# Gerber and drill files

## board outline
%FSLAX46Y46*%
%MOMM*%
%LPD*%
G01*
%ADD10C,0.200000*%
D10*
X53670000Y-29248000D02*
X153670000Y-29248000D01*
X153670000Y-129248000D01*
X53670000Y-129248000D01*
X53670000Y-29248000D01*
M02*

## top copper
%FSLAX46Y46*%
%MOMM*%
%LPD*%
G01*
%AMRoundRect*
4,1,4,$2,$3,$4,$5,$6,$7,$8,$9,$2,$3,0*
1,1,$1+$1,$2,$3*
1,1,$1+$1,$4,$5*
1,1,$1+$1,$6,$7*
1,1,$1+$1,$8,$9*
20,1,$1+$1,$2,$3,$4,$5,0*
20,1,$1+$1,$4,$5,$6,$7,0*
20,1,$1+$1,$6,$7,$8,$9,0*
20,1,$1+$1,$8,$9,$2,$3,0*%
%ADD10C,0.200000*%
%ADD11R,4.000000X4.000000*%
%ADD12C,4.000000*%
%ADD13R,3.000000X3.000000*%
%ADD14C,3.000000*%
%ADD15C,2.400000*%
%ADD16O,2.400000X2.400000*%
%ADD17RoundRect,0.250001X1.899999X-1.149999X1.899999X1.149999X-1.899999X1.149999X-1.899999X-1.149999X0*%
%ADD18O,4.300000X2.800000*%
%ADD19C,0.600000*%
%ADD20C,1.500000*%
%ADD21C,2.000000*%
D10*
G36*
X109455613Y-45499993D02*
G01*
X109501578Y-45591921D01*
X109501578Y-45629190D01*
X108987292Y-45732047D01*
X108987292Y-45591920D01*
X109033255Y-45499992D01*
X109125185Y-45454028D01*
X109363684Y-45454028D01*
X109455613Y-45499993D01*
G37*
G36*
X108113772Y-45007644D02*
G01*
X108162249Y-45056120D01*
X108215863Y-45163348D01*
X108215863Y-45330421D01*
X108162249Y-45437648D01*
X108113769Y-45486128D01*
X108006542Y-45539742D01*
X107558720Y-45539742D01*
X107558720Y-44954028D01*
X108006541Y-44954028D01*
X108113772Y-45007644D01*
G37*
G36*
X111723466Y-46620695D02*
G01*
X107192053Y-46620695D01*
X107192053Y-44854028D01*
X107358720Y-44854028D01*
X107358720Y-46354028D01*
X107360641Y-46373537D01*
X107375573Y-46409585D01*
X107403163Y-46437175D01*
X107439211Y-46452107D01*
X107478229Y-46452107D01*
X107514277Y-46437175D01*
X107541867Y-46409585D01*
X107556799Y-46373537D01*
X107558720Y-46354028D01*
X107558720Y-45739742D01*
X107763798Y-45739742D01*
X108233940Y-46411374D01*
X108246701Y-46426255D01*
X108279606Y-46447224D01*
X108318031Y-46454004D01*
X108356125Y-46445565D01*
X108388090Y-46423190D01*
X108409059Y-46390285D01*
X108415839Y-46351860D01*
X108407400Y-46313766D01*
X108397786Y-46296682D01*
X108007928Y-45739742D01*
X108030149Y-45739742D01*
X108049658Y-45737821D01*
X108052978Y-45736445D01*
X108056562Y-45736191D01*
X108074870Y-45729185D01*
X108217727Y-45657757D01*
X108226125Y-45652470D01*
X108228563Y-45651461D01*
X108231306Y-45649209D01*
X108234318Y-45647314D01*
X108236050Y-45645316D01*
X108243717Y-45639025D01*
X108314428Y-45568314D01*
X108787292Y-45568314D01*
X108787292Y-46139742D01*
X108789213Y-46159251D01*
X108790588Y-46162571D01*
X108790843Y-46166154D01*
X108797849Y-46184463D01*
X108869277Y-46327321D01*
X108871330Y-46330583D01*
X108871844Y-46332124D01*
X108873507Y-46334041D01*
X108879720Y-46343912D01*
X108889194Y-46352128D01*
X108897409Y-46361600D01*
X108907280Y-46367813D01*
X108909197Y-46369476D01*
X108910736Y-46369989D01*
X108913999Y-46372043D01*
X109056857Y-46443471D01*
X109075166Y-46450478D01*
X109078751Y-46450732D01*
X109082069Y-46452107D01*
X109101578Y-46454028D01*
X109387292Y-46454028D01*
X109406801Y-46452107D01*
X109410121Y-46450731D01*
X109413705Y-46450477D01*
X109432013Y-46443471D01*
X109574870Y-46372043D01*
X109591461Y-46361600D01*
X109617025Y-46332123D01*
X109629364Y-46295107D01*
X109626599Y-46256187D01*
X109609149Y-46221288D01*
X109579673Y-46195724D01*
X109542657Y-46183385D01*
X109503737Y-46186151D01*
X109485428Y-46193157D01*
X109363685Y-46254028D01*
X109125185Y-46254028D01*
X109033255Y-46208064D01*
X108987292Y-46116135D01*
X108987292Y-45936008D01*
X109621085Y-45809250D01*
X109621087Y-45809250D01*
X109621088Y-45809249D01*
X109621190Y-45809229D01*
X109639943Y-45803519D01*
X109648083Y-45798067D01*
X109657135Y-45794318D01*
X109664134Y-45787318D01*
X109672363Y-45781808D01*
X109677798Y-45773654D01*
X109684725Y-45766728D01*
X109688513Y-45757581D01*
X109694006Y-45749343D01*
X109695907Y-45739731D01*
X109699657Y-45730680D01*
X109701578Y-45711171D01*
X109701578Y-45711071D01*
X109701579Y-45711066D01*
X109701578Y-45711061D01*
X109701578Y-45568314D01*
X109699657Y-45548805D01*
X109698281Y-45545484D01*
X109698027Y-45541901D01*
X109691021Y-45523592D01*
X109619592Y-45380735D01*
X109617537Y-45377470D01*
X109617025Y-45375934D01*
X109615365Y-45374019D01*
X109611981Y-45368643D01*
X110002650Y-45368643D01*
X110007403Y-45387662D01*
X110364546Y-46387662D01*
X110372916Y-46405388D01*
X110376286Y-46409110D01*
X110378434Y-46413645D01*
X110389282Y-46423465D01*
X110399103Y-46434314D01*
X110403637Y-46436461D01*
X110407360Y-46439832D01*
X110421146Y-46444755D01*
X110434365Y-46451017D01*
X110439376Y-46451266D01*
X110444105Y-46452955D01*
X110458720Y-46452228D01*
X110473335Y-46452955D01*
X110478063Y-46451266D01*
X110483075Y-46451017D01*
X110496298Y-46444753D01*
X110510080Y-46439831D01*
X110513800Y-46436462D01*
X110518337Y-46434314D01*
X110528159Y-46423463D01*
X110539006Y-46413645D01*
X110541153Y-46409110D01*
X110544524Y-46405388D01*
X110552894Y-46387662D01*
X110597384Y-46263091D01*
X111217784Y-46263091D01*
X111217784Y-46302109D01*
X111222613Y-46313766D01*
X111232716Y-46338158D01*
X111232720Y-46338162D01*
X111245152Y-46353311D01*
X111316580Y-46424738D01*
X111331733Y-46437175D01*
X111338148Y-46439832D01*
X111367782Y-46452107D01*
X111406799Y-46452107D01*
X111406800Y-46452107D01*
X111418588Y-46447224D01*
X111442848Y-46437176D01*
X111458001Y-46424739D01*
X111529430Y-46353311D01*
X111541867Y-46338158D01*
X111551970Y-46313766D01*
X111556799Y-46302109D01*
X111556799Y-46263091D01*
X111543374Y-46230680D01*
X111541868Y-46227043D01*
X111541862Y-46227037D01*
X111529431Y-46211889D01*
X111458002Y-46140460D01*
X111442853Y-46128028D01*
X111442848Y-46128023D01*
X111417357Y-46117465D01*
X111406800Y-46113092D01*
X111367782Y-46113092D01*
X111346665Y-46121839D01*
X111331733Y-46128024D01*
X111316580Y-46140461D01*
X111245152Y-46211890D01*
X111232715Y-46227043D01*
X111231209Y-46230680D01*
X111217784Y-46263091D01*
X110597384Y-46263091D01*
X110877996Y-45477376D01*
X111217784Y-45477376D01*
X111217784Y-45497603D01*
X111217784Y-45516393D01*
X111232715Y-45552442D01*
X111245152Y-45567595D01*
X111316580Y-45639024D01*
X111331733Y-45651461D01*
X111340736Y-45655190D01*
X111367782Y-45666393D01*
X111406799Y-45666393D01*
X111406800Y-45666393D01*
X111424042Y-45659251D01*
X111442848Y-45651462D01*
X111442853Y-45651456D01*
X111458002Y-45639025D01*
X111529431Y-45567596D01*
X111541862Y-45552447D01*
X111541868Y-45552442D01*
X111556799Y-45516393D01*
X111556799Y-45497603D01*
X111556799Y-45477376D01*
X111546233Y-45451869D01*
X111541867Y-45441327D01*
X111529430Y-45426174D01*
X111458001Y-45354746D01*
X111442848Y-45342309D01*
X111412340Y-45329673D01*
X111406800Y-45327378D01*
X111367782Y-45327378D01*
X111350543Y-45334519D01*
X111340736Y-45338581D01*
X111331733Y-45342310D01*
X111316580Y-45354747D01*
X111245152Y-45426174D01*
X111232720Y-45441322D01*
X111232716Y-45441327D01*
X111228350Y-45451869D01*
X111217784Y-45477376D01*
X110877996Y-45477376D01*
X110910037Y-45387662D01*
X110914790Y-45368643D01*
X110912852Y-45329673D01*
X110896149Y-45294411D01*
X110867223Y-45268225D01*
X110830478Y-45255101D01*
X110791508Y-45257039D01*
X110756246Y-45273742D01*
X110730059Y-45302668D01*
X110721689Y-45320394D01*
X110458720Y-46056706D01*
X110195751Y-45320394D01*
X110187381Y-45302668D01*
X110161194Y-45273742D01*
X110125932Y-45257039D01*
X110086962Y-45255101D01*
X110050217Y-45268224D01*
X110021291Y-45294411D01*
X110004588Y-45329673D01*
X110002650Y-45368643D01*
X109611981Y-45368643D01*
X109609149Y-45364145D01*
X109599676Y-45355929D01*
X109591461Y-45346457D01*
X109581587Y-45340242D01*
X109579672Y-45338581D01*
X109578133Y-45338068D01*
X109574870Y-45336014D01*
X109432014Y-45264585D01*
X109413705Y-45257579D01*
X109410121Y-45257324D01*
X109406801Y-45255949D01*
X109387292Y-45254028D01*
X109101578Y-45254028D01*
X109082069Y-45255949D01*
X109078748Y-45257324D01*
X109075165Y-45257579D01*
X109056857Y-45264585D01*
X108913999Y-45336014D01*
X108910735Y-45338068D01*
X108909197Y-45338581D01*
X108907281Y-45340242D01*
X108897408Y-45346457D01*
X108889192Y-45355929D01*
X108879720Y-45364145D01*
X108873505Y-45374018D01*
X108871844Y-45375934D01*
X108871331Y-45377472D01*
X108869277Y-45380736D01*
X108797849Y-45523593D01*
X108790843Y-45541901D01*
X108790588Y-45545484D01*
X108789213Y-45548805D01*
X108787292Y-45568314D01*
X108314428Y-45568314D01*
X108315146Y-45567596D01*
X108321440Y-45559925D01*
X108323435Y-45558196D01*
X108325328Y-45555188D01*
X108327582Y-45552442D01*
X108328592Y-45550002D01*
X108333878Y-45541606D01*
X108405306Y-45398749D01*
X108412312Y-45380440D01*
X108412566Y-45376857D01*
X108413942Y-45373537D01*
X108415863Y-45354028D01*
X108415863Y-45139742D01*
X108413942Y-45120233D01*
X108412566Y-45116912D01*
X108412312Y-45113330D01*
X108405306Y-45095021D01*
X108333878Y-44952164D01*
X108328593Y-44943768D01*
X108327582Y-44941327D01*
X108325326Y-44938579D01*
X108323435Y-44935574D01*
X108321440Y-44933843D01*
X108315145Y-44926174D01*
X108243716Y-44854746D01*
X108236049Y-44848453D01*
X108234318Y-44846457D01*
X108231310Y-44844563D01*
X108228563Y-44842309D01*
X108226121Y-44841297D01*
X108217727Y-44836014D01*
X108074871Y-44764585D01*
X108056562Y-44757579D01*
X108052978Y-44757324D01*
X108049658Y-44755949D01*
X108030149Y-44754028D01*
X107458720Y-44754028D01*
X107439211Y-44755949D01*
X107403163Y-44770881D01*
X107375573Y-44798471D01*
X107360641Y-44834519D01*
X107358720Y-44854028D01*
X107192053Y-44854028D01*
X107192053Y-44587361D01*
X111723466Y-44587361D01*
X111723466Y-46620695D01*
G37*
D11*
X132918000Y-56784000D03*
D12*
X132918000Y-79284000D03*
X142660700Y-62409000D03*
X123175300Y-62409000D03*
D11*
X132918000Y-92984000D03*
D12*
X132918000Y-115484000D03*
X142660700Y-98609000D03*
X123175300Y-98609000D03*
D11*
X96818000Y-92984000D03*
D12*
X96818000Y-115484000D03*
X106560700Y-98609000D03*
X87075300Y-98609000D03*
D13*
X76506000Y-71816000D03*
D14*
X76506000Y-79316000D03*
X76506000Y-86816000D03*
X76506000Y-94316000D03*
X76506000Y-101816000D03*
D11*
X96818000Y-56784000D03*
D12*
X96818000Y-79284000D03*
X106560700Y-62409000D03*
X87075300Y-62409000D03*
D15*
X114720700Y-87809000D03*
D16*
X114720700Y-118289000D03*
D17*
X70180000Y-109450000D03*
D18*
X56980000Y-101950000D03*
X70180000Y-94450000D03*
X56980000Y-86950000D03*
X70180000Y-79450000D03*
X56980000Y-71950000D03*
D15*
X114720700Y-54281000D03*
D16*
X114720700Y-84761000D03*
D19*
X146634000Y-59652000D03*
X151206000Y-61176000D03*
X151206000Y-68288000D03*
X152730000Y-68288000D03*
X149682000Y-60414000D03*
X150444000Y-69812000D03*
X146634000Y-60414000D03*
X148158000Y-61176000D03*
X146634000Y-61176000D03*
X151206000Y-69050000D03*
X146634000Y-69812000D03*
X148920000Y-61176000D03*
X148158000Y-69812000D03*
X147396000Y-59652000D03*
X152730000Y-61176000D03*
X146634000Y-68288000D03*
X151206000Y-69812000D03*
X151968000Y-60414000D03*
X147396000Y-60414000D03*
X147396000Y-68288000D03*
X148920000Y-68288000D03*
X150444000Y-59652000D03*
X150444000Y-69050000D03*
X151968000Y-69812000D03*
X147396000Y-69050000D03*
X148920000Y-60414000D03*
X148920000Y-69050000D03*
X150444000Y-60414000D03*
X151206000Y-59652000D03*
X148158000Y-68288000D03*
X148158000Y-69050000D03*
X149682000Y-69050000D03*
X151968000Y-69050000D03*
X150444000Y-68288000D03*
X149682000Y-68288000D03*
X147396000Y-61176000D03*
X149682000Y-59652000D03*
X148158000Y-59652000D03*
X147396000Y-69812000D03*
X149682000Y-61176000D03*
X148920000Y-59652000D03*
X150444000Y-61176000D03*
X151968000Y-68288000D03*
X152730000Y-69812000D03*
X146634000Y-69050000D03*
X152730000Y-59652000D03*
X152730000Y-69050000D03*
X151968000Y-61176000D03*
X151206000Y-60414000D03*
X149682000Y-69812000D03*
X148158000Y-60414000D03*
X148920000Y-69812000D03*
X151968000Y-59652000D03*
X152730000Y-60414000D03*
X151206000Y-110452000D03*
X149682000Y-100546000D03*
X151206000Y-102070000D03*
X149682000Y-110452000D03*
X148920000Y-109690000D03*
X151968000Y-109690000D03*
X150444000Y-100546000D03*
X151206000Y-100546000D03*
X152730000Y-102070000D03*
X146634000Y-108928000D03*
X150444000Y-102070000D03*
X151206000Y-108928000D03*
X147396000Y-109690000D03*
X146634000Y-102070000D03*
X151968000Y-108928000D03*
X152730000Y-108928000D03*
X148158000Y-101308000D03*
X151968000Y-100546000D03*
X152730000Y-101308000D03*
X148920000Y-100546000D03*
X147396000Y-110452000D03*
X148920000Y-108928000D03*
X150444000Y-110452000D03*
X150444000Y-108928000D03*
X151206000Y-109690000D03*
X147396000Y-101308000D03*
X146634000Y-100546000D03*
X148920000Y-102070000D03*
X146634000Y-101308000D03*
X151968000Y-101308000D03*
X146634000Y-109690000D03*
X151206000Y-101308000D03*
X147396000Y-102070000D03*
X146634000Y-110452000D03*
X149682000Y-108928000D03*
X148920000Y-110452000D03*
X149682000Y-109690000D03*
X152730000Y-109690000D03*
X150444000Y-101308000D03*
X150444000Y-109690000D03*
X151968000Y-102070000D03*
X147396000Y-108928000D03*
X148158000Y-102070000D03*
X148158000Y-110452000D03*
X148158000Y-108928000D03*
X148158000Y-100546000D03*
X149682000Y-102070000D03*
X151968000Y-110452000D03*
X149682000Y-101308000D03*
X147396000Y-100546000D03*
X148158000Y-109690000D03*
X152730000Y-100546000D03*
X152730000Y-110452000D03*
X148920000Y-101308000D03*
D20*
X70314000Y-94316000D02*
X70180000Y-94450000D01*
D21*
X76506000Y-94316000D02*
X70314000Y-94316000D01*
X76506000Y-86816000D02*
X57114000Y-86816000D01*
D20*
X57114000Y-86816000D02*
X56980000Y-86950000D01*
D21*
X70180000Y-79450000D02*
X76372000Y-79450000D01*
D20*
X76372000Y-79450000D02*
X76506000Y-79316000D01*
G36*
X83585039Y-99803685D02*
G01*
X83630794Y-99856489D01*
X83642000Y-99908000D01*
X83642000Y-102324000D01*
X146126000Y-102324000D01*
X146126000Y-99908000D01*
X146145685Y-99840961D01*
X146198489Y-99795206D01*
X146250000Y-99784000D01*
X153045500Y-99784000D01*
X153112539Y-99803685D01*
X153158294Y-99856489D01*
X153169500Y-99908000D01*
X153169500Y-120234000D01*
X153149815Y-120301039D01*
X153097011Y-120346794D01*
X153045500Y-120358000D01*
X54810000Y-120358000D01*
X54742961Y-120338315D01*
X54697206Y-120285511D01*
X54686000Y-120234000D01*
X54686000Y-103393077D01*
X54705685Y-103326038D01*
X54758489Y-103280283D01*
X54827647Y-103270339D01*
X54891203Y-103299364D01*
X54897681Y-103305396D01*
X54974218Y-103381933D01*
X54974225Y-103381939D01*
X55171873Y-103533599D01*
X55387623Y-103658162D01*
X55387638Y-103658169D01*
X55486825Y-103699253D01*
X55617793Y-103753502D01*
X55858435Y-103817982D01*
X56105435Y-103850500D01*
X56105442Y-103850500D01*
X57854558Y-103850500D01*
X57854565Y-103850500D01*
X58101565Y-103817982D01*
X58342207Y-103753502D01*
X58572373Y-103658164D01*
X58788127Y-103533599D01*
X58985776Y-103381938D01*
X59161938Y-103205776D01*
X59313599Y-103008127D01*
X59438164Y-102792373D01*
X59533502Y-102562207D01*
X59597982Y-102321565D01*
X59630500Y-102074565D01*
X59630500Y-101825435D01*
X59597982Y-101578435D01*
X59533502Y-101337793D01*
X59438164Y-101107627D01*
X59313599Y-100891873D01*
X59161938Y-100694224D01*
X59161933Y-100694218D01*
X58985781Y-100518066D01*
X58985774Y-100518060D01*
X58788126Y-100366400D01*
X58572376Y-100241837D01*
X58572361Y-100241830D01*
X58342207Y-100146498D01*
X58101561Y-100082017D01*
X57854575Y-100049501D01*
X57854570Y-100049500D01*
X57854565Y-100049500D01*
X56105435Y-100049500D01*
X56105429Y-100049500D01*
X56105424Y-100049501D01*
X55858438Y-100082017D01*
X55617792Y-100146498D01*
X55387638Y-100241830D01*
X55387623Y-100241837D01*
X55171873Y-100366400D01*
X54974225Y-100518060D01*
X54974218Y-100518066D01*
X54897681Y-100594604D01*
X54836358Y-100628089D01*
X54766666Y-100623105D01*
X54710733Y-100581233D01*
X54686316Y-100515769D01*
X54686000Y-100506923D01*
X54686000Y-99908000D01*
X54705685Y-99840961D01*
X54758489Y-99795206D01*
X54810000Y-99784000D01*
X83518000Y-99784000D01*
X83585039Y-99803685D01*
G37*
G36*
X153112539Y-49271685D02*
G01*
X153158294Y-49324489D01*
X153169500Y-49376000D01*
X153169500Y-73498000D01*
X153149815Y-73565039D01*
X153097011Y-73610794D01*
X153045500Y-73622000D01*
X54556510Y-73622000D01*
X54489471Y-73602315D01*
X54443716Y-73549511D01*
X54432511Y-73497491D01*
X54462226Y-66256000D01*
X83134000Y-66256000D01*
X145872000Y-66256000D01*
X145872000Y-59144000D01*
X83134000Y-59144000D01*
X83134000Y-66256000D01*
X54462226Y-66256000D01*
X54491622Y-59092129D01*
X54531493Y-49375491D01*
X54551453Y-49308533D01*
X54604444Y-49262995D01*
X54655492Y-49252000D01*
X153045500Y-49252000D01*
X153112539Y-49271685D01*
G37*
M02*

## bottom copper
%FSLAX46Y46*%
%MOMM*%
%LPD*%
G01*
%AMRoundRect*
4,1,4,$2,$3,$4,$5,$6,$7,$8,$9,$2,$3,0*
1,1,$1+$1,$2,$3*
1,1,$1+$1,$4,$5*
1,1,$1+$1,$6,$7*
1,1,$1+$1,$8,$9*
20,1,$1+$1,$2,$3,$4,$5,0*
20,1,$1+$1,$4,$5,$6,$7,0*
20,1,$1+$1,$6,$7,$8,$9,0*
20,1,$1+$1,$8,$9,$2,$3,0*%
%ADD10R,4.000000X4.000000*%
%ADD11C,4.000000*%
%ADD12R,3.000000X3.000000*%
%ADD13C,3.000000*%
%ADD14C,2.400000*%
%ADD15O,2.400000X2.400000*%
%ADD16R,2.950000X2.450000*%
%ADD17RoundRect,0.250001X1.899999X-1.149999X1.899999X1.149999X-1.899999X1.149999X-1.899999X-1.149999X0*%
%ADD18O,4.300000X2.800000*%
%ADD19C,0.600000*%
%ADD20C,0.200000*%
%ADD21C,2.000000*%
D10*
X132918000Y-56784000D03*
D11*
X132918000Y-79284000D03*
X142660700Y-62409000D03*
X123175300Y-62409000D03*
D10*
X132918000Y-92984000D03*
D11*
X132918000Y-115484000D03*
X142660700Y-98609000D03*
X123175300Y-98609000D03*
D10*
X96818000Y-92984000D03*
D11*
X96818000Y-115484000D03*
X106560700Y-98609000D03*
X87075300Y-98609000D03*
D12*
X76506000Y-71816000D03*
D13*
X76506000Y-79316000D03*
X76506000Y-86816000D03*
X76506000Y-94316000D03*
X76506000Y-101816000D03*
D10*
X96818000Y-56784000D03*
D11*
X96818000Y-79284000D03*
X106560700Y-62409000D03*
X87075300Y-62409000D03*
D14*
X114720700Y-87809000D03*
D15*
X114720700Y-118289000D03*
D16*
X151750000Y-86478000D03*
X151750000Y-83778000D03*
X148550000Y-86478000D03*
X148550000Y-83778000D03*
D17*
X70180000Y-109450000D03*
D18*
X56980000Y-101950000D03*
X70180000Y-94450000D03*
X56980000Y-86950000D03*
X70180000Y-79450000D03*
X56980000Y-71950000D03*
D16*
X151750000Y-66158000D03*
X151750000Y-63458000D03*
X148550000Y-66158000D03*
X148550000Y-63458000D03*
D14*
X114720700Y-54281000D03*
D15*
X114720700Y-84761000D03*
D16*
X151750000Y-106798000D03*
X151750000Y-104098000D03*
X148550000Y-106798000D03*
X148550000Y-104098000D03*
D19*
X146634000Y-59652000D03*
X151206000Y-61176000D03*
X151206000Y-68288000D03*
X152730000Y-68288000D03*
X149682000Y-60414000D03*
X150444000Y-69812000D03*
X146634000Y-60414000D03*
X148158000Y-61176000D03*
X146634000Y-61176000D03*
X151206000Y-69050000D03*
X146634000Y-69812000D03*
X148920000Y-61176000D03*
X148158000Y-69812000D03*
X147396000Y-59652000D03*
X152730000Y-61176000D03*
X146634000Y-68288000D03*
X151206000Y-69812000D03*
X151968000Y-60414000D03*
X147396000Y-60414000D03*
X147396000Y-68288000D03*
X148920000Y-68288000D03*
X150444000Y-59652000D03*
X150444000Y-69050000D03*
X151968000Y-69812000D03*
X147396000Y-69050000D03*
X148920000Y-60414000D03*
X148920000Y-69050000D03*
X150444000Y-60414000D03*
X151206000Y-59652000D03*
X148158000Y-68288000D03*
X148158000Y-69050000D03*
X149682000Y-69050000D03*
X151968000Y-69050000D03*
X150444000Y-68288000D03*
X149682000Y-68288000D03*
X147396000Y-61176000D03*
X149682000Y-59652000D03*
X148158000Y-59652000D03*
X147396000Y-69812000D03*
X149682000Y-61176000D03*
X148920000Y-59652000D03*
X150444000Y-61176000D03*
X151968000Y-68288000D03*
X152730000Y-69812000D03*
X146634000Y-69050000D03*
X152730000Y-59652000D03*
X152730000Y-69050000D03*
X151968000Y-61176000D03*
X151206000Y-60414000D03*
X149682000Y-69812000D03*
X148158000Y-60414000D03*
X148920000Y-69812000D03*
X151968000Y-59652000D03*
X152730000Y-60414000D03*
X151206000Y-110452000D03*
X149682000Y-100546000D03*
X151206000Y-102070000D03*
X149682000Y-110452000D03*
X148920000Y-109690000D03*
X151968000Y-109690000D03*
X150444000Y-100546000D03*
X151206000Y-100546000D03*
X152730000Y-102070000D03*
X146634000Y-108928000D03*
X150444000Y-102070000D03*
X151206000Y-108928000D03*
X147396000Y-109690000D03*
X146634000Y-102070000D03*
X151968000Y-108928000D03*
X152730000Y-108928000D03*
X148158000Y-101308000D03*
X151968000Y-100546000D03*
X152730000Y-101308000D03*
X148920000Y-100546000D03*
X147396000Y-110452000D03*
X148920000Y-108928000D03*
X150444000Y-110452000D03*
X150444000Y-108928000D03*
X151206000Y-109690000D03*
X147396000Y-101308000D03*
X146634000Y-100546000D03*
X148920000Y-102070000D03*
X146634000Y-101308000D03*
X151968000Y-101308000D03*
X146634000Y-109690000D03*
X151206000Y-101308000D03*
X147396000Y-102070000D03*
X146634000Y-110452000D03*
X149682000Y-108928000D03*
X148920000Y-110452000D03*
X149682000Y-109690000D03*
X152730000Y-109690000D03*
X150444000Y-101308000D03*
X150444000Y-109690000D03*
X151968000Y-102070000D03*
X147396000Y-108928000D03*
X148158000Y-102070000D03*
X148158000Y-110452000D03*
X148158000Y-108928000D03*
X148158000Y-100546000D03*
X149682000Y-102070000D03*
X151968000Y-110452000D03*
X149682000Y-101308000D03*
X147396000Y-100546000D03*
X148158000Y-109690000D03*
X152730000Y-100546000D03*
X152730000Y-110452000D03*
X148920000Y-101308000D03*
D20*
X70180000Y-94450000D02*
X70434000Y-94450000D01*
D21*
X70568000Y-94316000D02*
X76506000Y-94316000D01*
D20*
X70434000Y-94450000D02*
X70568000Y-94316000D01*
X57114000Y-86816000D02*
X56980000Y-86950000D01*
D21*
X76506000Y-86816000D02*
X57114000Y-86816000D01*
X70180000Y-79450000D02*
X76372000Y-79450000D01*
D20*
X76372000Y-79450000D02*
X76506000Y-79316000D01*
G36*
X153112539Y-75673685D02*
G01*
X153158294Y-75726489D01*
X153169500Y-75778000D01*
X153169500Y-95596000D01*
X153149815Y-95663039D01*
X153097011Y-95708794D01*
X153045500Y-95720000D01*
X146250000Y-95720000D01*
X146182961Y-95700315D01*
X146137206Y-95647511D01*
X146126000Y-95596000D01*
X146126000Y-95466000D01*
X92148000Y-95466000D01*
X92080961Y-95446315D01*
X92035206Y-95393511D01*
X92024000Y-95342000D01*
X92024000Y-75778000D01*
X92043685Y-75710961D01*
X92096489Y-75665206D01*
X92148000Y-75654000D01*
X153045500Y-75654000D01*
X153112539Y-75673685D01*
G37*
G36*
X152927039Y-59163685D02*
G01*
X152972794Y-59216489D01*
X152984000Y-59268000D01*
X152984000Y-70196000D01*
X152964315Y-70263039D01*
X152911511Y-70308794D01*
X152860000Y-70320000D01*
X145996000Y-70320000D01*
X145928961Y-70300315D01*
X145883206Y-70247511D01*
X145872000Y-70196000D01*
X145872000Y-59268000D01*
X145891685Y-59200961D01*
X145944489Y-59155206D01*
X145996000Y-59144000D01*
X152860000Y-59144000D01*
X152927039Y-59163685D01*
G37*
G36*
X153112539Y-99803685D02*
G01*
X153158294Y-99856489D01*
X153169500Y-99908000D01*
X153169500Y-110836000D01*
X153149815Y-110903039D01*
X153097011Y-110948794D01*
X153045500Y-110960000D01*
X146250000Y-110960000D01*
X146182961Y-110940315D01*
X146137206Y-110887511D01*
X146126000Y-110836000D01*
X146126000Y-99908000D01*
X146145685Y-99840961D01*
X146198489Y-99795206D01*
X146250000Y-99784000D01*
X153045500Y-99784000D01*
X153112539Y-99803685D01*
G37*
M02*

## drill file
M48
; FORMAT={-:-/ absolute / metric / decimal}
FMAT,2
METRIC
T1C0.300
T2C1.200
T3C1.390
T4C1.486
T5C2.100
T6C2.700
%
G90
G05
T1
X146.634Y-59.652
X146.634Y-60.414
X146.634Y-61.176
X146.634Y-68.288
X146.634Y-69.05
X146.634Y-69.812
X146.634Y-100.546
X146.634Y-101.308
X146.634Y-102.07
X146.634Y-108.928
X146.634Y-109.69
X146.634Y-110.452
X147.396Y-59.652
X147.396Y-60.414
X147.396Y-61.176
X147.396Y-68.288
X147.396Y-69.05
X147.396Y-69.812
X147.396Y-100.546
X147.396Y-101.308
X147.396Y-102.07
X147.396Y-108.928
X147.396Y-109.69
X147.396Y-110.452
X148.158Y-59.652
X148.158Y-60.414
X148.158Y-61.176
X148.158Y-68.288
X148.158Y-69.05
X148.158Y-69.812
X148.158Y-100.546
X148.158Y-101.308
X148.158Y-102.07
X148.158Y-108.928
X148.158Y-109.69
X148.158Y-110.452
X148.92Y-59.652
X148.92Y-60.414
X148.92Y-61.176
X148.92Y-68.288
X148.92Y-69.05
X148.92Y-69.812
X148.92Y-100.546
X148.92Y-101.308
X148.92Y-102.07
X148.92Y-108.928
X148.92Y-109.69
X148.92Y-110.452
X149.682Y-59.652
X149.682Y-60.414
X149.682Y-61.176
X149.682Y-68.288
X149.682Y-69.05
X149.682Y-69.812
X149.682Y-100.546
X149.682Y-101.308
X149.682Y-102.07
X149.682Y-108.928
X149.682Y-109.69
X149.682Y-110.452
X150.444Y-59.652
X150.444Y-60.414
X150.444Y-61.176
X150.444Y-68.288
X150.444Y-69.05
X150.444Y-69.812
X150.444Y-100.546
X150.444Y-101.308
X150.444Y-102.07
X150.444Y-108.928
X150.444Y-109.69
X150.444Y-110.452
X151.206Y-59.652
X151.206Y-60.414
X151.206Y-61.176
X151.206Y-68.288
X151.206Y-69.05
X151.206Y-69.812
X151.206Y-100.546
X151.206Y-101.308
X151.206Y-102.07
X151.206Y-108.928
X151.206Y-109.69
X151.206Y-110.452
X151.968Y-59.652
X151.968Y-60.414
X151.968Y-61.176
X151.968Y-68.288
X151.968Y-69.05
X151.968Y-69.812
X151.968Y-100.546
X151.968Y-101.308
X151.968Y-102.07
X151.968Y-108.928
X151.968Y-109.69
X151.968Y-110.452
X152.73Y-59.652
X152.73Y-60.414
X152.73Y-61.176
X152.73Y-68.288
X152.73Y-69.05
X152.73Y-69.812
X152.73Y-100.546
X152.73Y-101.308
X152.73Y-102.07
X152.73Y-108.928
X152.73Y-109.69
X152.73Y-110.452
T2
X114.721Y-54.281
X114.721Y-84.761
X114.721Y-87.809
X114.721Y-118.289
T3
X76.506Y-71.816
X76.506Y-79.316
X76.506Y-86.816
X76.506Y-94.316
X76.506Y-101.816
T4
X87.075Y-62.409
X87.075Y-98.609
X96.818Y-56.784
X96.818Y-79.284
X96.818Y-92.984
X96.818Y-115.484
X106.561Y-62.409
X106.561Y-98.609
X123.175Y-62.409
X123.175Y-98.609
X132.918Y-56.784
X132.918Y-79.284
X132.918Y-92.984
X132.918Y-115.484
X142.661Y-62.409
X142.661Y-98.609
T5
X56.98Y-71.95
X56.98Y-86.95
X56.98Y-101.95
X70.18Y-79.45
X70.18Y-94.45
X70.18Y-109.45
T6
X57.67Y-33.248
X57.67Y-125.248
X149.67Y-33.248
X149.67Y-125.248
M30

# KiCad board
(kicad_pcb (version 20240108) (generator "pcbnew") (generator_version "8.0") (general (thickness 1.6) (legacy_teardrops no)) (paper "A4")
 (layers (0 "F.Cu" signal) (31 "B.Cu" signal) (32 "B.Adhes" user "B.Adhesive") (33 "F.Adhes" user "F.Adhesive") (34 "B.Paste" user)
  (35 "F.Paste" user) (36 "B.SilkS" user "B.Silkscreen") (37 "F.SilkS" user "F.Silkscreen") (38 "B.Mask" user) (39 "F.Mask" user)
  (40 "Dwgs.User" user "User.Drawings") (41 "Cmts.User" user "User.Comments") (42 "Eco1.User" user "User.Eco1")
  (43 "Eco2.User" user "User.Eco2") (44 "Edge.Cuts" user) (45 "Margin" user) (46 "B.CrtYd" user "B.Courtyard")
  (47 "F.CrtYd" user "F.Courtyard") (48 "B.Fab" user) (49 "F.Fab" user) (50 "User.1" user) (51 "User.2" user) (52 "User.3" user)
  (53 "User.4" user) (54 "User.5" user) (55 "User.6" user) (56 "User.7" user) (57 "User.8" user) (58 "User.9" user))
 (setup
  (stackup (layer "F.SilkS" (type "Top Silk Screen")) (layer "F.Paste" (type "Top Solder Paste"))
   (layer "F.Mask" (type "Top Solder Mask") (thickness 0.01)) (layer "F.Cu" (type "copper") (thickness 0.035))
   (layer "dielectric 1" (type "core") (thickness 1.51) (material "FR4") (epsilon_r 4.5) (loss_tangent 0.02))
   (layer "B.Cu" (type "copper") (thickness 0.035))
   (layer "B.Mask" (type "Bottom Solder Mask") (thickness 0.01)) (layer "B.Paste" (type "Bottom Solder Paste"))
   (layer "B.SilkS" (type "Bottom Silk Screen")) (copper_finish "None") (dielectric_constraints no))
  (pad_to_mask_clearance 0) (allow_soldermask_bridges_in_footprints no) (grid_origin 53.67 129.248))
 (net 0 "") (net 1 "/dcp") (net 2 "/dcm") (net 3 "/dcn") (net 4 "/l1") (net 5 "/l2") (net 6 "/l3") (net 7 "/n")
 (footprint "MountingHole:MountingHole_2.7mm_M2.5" (layer "F.Cu") (at 57.67 125.248 -90)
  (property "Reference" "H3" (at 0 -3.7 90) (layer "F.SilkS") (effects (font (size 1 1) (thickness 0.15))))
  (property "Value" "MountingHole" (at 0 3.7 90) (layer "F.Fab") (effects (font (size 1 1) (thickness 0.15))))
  (pad "" np_thru_hole circle (at 0 0 270) (size 2.7 2.7) (drill 2.7) (layers "*.Cu" "*.Mask")))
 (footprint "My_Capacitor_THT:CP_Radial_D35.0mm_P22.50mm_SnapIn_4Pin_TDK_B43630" (layer "F.Cu") (at 132.918 56.784 -90)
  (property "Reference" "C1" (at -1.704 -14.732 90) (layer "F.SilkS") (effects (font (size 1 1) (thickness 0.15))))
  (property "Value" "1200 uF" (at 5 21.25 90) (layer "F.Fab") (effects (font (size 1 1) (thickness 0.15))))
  (pad "1" thru_hole rect (at 0 0 270) (size 4 4) (drill 1.486) (layers "*.Cu" "*.Mask") (remove_unused_layers no) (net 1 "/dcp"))
  (pad "2" thru_hole circle (at 22.5 0 270) (size 4 4) (drill 1.486) (layers "*.Cu" "*.Mask") (remove_unused_layers no) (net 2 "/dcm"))
  (pad "SH" thru_hole circle (at 5.625 -9.7427 270) (size 4 4) (drill 1.486) (layers "*.Cu" "*.Mask") (remove_unused_layers no))
  (pad "SH" thru_hole circle (at 5.625 9.7427 270) (size 4 4) (drill 1.486) (layers "*.Cu" "*.Mask") (remove_unused_layers no)))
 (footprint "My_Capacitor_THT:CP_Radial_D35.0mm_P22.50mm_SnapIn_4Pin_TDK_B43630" (layer "F.Cu") (at 132.918 92.984 -90)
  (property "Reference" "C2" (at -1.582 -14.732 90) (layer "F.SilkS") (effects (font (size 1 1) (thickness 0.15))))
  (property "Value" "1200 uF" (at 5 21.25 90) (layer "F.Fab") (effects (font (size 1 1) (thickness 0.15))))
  (pad "1" thru_hole rect (at 0 0 270) (size 4 4) (drill 1.486) (layers "*.Cu" "*.Mask") (remove_unused_layers no) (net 2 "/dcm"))
  (pad "2" thru_hole circle (at 22.5 0 270) (size 4 4) (drill 1.486) (layers "*.Cu" "*.Mask") (remove_unused_layers no) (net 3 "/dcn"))
  (pad "SH" thru_hole circle (at 5.625 -9.7427 270) (size 4 4) (drill 1.486) (layers "*.Cu" "*.Mask") (remove_unused_layers no))
  (pad "SH" thru_hole circle (at 5.625 9.7427 270) (size 4 4) (drill 1.486) (layers "*.Cu" "*.Mask") (remove_unused_layers no)))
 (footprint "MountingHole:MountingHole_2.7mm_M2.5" (layer "F.Cu") (at 149.67 33.248 180)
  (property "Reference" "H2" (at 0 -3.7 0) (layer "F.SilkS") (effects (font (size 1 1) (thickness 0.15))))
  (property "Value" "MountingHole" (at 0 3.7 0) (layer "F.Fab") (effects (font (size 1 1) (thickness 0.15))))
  (pad "" np_thru_hole circle (at 0 0 180) (size 2.7 2.7) (drill 2.7) (layers "*.Cu" "*.Mask")))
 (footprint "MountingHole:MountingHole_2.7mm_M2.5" (layer "F.Cu") (at 149.67 125.248 90)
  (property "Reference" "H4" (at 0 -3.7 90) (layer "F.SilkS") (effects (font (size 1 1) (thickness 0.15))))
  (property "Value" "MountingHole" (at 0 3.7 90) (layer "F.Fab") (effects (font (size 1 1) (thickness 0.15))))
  (pad "" np_thru_hole circle (at 0 0 90) (size 2.7 2.7) (drill 2.7) (layers "*.Cu" "*.Mask")))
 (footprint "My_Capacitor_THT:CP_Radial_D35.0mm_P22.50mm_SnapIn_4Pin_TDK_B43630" (layer "F.Cu") (at 96.818 92.984 -90)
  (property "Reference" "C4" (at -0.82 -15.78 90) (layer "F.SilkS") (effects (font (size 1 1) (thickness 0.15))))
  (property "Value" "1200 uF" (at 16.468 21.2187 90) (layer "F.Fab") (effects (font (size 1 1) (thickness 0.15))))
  (pad "1" thru_hole rect (at 0 0 270) (size 4 4) (drill 1.486) (layers "*.Cu" "*.Mask") (remove_unused_layers no) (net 2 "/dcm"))
  (pad "2" thru_hole circle (at 22.5 0 270) (size 4 4) (drill 1.486) (layers "*.Cu" "*.Mask") (remove_unused_layers no) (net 3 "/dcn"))
  (pad "SH" thru_hole circle (at 5.625 -9.7427 270) (size 4 4) (drill 1.486) (layers "*.Cu" "*.Mask") (remove_unused_layers no))
  (pad "SH" thru_hole circle (at 5.625 9.7427 270) (size 4 4) (drill 1.486) (layers "*.Cu" "*.Mask") (remove_unused_layers no)))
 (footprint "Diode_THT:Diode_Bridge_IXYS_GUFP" (layer "F.Cu") (at 76.506 71.816)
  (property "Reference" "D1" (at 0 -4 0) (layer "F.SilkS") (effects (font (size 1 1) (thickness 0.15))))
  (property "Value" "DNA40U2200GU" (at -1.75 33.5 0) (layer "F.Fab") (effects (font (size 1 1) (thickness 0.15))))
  (pad "1" thru_hole rect (at 0 0) (size 3 3) (drill 1.39) (layers "*.Cu" "*.Mask") (remove_unused_layers no) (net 1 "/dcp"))
  (pad "2" thru_hole circle (at 0 7.5) (size 3 3) (drill 1.39) (layers "*.Cu" "*.Mask") (remove_unused_layers no) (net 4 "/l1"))
  (pad "3" thru_hole circle (at 0 15) (size 3 3) (drill 1.39) (layers "*.Cu" "*.Mask") (remove_unused_layers no) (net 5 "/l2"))
  (pad "4" thru_hole circle (at 0 22.5) (size 3 3) (drill 1.39) (layers "*.Cu" "*.Mask") (remove_unused_layers no) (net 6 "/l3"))
  (pad "5" thru_hole circle (at 0 30) (size 3 3) (drill 1.39) (layers "*.Cu" "*.Mask") (remove_unused_layers no) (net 3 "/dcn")))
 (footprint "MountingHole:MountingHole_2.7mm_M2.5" (layer "F.Cu") (at 57.67 33.248 180)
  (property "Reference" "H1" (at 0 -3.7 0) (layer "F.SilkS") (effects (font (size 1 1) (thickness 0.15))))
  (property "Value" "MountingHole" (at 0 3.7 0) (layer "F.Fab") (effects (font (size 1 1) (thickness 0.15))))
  (pad "" np_thru_hole circle (at 0 0 180) (size 2.7 2.7) (drill 2.7) (layers "*.Cu" "*.Mask")))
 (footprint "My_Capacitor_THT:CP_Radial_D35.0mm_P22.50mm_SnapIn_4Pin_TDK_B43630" (layer "F.Cu") (at 96.818 56.784 -90)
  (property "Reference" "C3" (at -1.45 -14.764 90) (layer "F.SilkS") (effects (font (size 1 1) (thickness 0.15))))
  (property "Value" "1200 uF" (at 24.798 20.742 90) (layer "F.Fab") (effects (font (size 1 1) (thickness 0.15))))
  (pad "1" thru_hole rect (at 0 0 270) (size 4 4) (drill 1.486) (layers "*.Cu" "*.Mask") (remove_unused_layers no) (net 1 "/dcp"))
  (pad "2" thru_hole circle (at 22.5 0 270) (size 4 4) (drill 1.486) (layers "*.Cu" "*.Mask") (remove_unused_layers no) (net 2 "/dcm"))
  (pad "SH" thru_hole circle (at 5.625 -9.7427 270) (size 4 4) (drill 1.486) (layers "*.Cu" "*.Mask") (remove_unused_layers no))
  (pad "SH" thru_hole circle (at 5.625 9.7427 270) (size 4 4) (drill 1.486) (layers "*.Cu" "*.Mask") (remove_unused_layers no)))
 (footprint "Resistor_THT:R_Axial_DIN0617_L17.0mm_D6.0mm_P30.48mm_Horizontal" (layer "B.Cu") (at 114.7207 87.809 -90)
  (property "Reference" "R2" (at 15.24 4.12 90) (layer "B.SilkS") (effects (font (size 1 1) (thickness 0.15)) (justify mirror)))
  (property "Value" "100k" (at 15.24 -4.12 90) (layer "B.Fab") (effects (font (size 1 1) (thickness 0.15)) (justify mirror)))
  (pad "1" thru_hole circle (at 0 0 270) (size 2.4 2.4) (drill 1.2) (layers "*.Cu" "*.Mask") (remove_unused_layers no) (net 2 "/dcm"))
  (pad "2" thru_hole oval (at 30.48 0 270) (size 2.4 2.4) (drill 1.2) (layers "*.Cu" "*.Mask") (remove_unused_layers no) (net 3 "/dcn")))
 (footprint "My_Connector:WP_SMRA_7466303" (layer "B.Cu") (at 150.15 85.128 180)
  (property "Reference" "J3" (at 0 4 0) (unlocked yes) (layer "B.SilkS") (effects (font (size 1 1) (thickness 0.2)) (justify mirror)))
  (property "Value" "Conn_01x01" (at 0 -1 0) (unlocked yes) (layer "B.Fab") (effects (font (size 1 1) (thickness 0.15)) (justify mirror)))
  (pad "1" smd rect (at -1.6 -1.35 180) (size 2.95 2.45) (layers "B.Cu" "B.Paste" "B.Mask") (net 2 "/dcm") (solder_mask_margin 0.125)
   (solder_paste_margin -0.2) (thermal_bridge_angle 45))
  (pad "1" smd rect (at -1.6 1.35 180) (size 2.95 2.45) (layers "B.Cu" "B.Paste" "B.Mask") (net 2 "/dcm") (solder_mask_margin 0.125)
   (solder_paste_margin -0.2) (thermal_bridge_angle 45))
  (pad "1" smd rect (at 1.6 -1.35 180) (size 2.95 2.45) (layers "B.Cu" "B.Paste" "B.Mask") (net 2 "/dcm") (solder_mask_margin 0.125)
   (solder_paste_margin -0.2) (thermal_bridge_angle 45))
  (pad "1" smd rect (at 1.6 1.35 180) (size 2.95 2.45) (layers "B.Cu" "B.Paste" "B.Mask") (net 2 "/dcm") (solder_mask_margin 0.125)
   (solder_paste_margin -0.2) (thermal_bridge_angle 45)))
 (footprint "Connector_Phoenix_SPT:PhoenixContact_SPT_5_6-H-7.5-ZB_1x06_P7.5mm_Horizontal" (layer "B.Cu") (at 70.18 109.45 90)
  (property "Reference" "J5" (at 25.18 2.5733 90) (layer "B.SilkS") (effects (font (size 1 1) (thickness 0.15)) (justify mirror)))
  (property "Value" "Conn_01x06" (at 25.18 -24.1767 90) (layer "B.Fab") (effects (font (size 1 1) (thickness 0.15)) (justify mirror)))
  (pad "1" thru_hole roundrect (at 0 0 90) (size 2.8 4.3) (drill 2.1) (layers "*.Cu" "*.Mask") (remove_unused_layers no)
   (roundrect_rratio 0.089286) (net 3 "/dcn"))
  (pad "2" thru_hole oval (at 7.5 -13.2 90) (size 2.8 4.3) (drill 2.1) (layers "*.Cu" "*.Mask") (remove_unused_layers no) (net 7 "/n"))
  (pad "3" thru_hole oval (at 15 0 90) (size 2.8 4.3) (drill 2.1) (layers "*.Cu" "*.Mask") (remove_unused_layers no) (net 6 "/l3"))
  (pad "4" thru_hole oval (at 22.5 -13.2 90) (size 2.8 4.3) (drill 2.1) (layers "*.Cu" "*.Mask") (remove_unused_layers no) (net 5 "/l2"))
  (pad "5" thru_hole oval (at 30 0 90) (size 2.8 4.3) (drill 2.1) (layers "*.Cu" "*.Mask") (remove_unused_layers no) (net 4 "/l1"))
  (pad "6" thru_hole oval (at 37.5 -13.2 90) (size 2.8 4.3) (drill 2.1) (layers "*.Cu" "*.Mask") (remove_unused_layers no) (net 1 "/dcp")))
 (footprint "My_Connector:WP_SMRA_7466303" (layer "B.Cu") (at 150.15 64.808 180)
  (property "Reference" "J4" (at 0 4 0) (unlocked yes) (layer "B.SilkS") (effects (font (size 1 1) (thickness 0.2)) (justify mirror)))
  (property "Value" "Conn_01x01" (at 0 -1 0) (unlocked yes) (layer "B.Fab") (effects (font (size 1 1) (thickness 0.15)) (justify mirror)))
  (pad "1" smd rect (at -1.6 -1.35 180) (size 2.95 2.45) (layers "B.Cu" "B.Paste" "B.Mask") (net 1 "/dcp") (solder_mask_margin 0.125)
   (solder_paste_margin -0.2) (thermal_bridge_angle 45))
  (pad "1" smd rect (at -1.6 1.35 180) (size 2.95 2.45) (layers "B.Cu" "B.Paste" "B.Mask") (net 1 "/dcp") (solder_mask_margin 0.125)
   (solder_paste_margin -0.2) (thermal_bridge_angle 45))
  (pad "1" smd rect (at 1.6 -1.35 180) (size 2.95 2.45) (layers "B.Cu" "B.Paste" "B.Mask") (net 1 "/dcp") (solder_mask_margin 0.125)
   (solder_paste_margin -0.2) (thermal_bridge_angle 45))
  (pad "1" smd rect (at 1.6 1.35 180) (size 2.95 2.45) (layers "B.Cu" "B.Paste" "B.Mask") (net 1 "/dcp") (solder_mask_margin 0.125)
   (solder_paste_margin -0.2) (thermal_bridge_angle 45)))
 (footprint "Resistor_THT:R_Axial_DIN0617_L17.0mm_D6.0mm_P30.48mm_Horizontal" (layer "B.Cu") (at 114.7207 54.281 -90)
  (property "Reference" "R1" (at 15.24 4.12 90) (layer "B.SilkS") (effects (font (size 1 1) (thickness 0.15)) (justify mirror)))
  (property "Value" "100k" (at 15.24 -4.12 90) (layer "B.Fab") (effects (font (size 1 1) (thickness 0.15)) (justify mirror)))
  (pad "1" thru_hole circle (at 0 0 270) (size 2.4 2.4) (drill 1.2) (layers "*.Cu" "*.Mask") (remove_unused_layers no) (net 1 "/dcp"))
  (pad "2" thru_hole oval (at 30.48 0 270) (size 2.4 2.4) (drill 1.2) (layers "*.Cu" "*.Mask") (remove_unused_layers no) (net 2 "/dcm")))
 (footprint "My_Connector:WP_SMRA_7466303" (layer "B.Cu") (at 150.15 105.448 180)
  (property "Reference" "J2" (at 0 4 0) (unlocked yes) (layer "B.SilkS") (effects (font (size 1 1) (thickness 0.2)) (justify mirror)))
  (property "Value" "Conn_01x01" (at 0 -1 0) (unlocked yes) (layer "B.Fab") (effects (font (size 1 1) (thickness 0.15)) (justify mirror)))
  (pad "1" smd rect (at -1.6 -1.35 180) (size 2.95 2.45) (layers "B.Cu" "B.Paste" "B.Mask") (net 3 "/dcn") (solder_mask_margin 0.125)
   (solder_paste_margin -0.2) (thermal_bridge_angle 45))
  (pad "1" smd rect (at -1.6 1.35 180) (size 2.95 2.45) (layers "B.Cu" "B.Paste" "B.Mask") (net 3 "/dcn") (solder_mask_margin 0.125)
   (solder_paste_margin -0.2) (thermal_bridge_angle 45))
  (pad "1" smd rect (at 1.6 -1.35 180) (size 2.95 2.45) (layers "B.Cu" "B.Paste" "B.Mask") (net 3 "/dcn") (solder_mask_margin 0.125)
   (solder_paste_margin -0.2) (thermal_bridge_angle 45))
  (pad "1" smd rect (at 1.6 1.35 180) (size 2.95 2.45) (layers "B.Cu" "B.Paste" "B.Mask") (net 3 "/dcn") (solder_mask_margin 0.125)
   (solder_paste_margin -0.2) (thermal_bridge_angle 45)))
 (gr_rect (start 53.67 29.248) (end 153.67 129.248) (stroke (width 0.2) (type default)) (fill none) (layer "Edge.Cuts"))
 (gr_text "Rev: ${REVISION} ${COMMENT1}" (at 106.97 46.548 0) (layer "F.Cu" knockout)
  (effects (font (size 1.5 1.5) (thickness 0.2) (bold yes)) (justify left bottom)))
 (segment (start 70.314 94.316) (end 70.18 94.45) (width 1.5) (layer "F.Cu") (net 6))
 (segment (start 76.506 94.316) (end 70.314 94.316) (width 2) (layer "F.Cu") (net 6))
 (segment (start 70.18 94.45) (end 70.434 94.45) (width 0.2) (layer "B.Cu") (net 6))
 (segment (start 70.568 94.316) (end 76.506 94.316) (width 2) (layer "B.Cu") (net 6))
 (segment (start 70.434 94.45) (end 70.568 94.316) (width 0.2) (layer "B.Cu") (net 6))
 (via (at 146.634 59.652) (size 0.6) (drill 0.3) (layers "F.Cu" "B.Cu") (free yes) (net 1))
 (via (at 151.206 61.176) (size 0.6) (drill 0.3) (layers "F.Cu" "B.Cu") (free yes) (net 1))
 (via (at 151.206 68.288) (size 0.6) (drill 0.3) (layers "F.Cu" "B.Cu") (free yes) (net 1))
 (via (at 152.73 68.288) (size 0.6) (drill 0.3) (layers "F.Cu" "B.Cu") (free yes) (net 1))
 (via (at 149.682 60.414) (size 0.6) (drill 0.3) (layers "F.Cu" "B.Cu") (free yes) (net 1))
 (via (at 150.444 69.812) (size 0.6) (drill 0.3) (layers "F.Cu" "B.Cu") (free yes) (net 1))
 (via (at 146.634 60.414) (size 0.6) (drill 0.3) (layers "F.Cu" "B.Cu") (free yes) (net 1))
 (via (at 148.158 61.176) (size 0.6) (drill 0.3) (layers "F.Cu" "B.Cu") (free yes) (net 1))
 (via (at 146.634 61.176) (size 0.6) (drill 0.3) (layers "F.Cu" "B.Cu") (free yes) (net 1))
 (via (at 151.206 69.05) (size 0.6) (drill 0.3) (layers "F.Cu" "B.Cu") (free yes) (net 1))
 (via (at 146.634 69.812) (size 0.6) (drill 0.3) (layers "F.Cu" "B.Cu") (free yes) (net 1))
 (via (at 148.92 61.176) (size 0.6) (drill 0.3) (layers "F.Cu" "B.Cu") (free yes) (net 1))
 (via (at 148.158 69.812) (size 0.6) (drill 0.3) (layers "F.Cu" "B.Cu") (free yes) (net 1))
 (via (at 147.396 59.652) (size 0.6) (drill 0.3) (layers "F.Cu" "B.Cu") (free yes) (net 1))
 (via (at 152.73 61.176) (size 0.6) (drill 0.3) (layers "F.Cu" "B.Cu") (free yes) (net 1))
 (via (at 146.634 68.288) (size 0.6) (drill 0.3) (layers "F.Cu" "B.Cu") (free yes) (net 1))
 (via (at 151.206 69.812) (size 0.6) (drill 0.3) (layers "F.Cu" "B.Cu") (free yes) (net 1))
 (via (at 151.968 60.414) (size 0.6) (drill 0.3) (layers "F.Cu" "B.Cu") (free yes) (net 1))
 (via (at 147.396 60.414) (size 0.6) (drill 0.3) (layers "F.Cu" "B.Cu") (free yes) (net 1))
 (via (at 147.396 68.288) (size 0.6) (drill 0.3) (layers "F.Cu" "B.Cu") (free yes) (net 1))
 (via (at 148.92 68.288) (size 0.6) (drill 0.3) (layers "F.Cu" "B.Cu") (free yes) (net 1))
 (via (at 150.444 59.652) (size 0.6) (drill 0.3) (layers "F.Cu" "B.Cu") (free yes) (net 1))
 (via (at 150.444 69.05) (size 0.6) (drill 0.3) (layers "F.Cu" "B.Cu") (free yes) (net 1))
 (via (at 151.968 69.812) (size 0.6) (drill 0.3) (layers "F.Cu" "B.Cu") (free yes) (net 1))
 (via (at 147.396 69.05) (size 0.6) (drill 0.3) (layers "F.Cu" "B.Cu") (free yes) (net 1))
 (via (at 148.92 60.414) (size 0.6) (drill 0.3) (layers "F.Cu" "B.Cu") (free yes) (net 1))
 (via (at 148.92 69.05) (size 0.6) (drill 0.3) (layers "F.Cu" "B.Cu") (free yes) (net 1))
 (via (at 150.444 60.414) (size 0.6) (drill 0.3) (layers "F.Cu" "B.Cu") (free yes) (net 1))
 (via (at 151.206 59.652) (size 0.6) (drill 0.3) (layers "F.Cu" "B.Cu") (free yes) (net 1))
 (via (at 148.158 68.288) (size 0.6) (drill 0.3) (layers "F.Cu" "B.Cu") (free yes) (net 1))
 (via (at 148.158 69.05) (size 0.6) (drill 0.3) (layers "F.Cu" "B.Cu") (free yes) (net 1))
 (via (at 149.682 69.05) (size 0.6) (drill 0.3) (layers "F.Cu" "B.Cu") (free yes) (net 1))
 (via (at 151.968 69.05) (size 0.6) (drill 0.3) (layers "F.Cu" "B.Cu") (free yes) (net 1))
 (via (at 150.444 68.288) (size 0.6) (drill 0.3) (layers "F.Cu" "B.Cu") (free yes) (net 1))
 (via (at 149.682 68.288) (size 0.6) (drill 0.3) (layers "F.Cu" "B.Cu") (free yes) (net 1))
 (via (at 147.396 61.176) (size 0.6) (drill 0.3) (layers "F.Cu" "B.Cu") (free yes) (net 1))
 (via (at 149.682 59.652) (size 0.6) (drill 0.3) (layers "F.Cu" "B.Cu") (free yes) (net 1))
 (via (at 148.158 59.652) (size 0.6) (drill 0.3) (layers "F.Cu" "B.Cu") (free yes) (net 1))
 (via (at 147.396 69.812) (size 0.6) (drill 0.3) (layers "F.Cu" "B.Cu") (free yes) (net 1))
 (via (at 149.682 61.176) (size 0.6) (drill 0.3) (layers "F.Cu" "B.Cu") (free yes) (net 1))
 (via (at 148.92 59.652) (size 0.6) (drill 0.3) (layers "F.Cu" "B.Cu") (free yes) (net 1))
 (via (at 150.444 61.176) (size 0.6) (drill 0.3) (layers "F.Cu" "B.Cu") (free yes) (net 1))
 (via (at 151.968 68.288) (size 0.6) (drill 0.3) (layers "F.Cu" "B.Cu") (free yes) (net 1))
 (via (at 152.73 69.812) (size 0.6) (drill 0.3) (layers "F.Cu" "B.Cu") (free yes) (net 1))
 (via (at 146.634 69.05) (size 0.6) (drill 0.3) (layers "F.Cu" "B.Cu") (free yes) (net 1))
 (via (at 152.73 59.652) (size 0.6) (drill 0.3) (layers "F.Cu" "B.Cu") (free yes) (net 1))
 (via (at 152.73 69.05) (size 0.6) (drill 0.3) (layers "F.Cu" "B.Cu") (free yes) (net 1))
 (via (at 151.968 61.176) (size 0.6) (drill 0.3) (layers "F.Cu" "B.Cu") (free yes) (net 1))
 (via (at 151.206 60.414) (size 0.6) (drill 0.3) (layers "F.Cu" "B.Cu") (free yes) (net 1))
 (via (at 149.682 69.812) (size 0.6) (drill 0.3) (layers "F.Cu" "B.Cu") (free yes) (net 1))
 (via (at 148.158 60.414) (size 0.6) (drill 0.3) (layers "F.Cu" "B.Cu") (free yes) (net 1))
 (via (at 148.92 69.812) (size 0.6) (drill 0.3) (layers "F.Cu" "B.Cu") (free yes) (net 1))
 (via (at 151.968 59.652) (size 0.6) (drill 0.3) (layers "F.Cu" "B.Cu") (free yes) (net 1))
 (via (at 152.73 60.414) (size 0.6) (drill 0.3) (layers "F.Cu" "B.Cu") (free yes) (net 1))
 (segment (start 76.506 86.816) (end 57.114 86.816) (width 2) (layer "F.Cu") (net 5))
 (segment (start 57.114 86.816) (end 56.98 86.95) (width 1.5) (layer "F.Cu") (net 5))
 (segment (start 57.114 86.816) (end 56.98 86.95) (width 0.2) (layer "B.Cu") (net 5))
 (segment (start 76.506 86.816) (end 57.114 86.816) (width 2) (layer "B.Cu") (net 5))
 (via (at 151.206 110.452) (size 0.6) (drill 0.3) (layers "F.Cu" "B.Cu") (free yes) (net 3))
 (via (at 149.682 100.546) (size 0.6) (drill 0.3) (layers "F.Cu" "B.Cu") (free yes) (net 3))
 (via (at 151.206 102.07) (size 0.6) (drill 0.3) (layers "F.Cu" "B.Cu") (free yes) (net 3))
 (via (at 149.682 110.452) (size 0.6) (drill 0.3) (layers "F.Cu" "B.Cu") (free yes) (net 3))
 (via (at 148.92 109.69) (size 0.6) (drill 0.3) (layers "F.Cu" "B.Cu") (free yes) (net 3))
 (via (at 151.968 109.69) (size 0.6) (drill 0.3) (layers "F.Cu" "B.Cu") (free yes) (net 3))
 (via (at 150.444 100.546) (size 0.6) (drill 0.3) (layers "F.Cu" "B.Cu") (free yes) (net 3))
 (via (at 151.206 100.546) (size 0.6) (drill 0.3) (layers "F.Cu" "B.Cu") (free yes) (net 3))
 (via (at 152.73 102.07) (size 0.6) (drill 0.3) (layers "F.Cu" "B.Cu") (free yes) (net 3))
 (via (at 146.634 108.928) (size 0.6) (drill 0.3) (layers "F.Cu" "B.Cu") (free yes) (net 3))
 (via (at 150.444 102.07) (size 0.6) (drill 0.3) (layers "F.Cu" "B.Cu") (free yes) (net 3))
 (via (at 151.206 108.928) (size 0.6) (drill 0.3) (layers "F.Cu" "B.Cu") (free yes) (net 3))
 (via (at 147.396 109.69) (size 0.6) (drill 0.3) (layers "F.Cu" "B.Cu") (free yes) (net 3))
 (via (at 146.634 102.07) (size 0.6) (drill 0.3) (layers "F.Cu" "B.Cu") (free yes) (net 3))
 (via (at 151.968 108.928) (size 0.6) (drill 0.3) (layers "F.Cu" "B.Cu") (free yes) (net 3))
 (via (at 152.73 108.928) (size 0.6) (drill 0.3) (layers "F.Cu" "B.Cu") (free yes) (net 3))
 (via (at 148.158 101.308) (size 0.6) (drill 0.3) (layers "F.Cu" "B.Cu") (free yes) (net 3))
 (via (at 151.968 100.546) (size 0.6) (drill 0.3) (layers "F.Cu" "B.Cu") (free yes) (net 3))
 (via (at 152.73 101.308) (size 0.6) (drill 0.3) (layers "F.Cu" "B.Cu") (free yes) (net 3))
 (via (at 148.92 100.546) (size 0.6) (drill 0.3) (layers "F.Cu" "B.Cu") (free yes) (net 3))
 (via (at 147.396 110.452) (size 0.6) (drill 0.3) (layers "F.Cu" "B.Cu") (free yes) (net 3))
 (via (at 148.92 108.928) (size 0.6) (drill 0.3) (layers "F.Cu" "B.Cu") (free yes) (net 3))
 (via (at 150.444 110.452) (size 0.6) (drill 0.3) (layers "F.Cu" "B.Cu") (free yes) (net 3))
 (via (at 150.444 108.928) (size 0.6) (drill 0.3) (layers "F.Cu" "B.Cu") (free yes) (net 3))
 (via (at 151.206 109.69) (size 0.6) (drill 0.3) (layers "F.Cu" "B.Cu") (free yes) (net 3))
 (via (at 147.396 101.308) (size 0.6) (drill 0.3) (layers "F.Cu" "B.Cu") (free yes) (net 3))
 (via (at 146.634 100.546) (size 0.6) (drill 0.3) (layers "F.Cu" "B.Cu") (free yes) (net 3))
 (via (at 148.92 102.07) (size 0.6) (drill 0.3) (layers "F.Cu" "B.Cu") (free yes) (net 3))
 (via (at 146.634 101.308) (size 0.6) (drill 0.3) (layers "F.Cu" "B.Cu") (free yes) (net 3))
 (via (at 151.968 101.308) (size 0.6) (drill 0.3) (layers "F.Cu" "B.Cu") (free yes) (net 3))
 (via (at 146.634 109.69) (size 0.6) (drill 0.3) (layers "F.Cu" "B.Cu") (free yes) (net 3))
 (via (at 151.206 101.308) (size 0.6) (drill 0.3) (layers "F.Cu" "B.Cu") (free yes) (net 3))
 (via (at 147.396 102.07) (size 0.6) (drill 0.3) (layers "F.Cu" "B.Cu") (free yes) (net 3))
 (via (at 146.634 110.452) (size 0.6) (drill 0.3) (layers "F.Cu" "B.Cu") (free yes) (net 3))
 (via (at 149.682 108.928) (size 0.6) (drill 0.3) (layers "F.Cu" "B.Cu") (free yes) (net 3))
 (via (at 148.92 110.452) (size 0.6) (drill 0.3) (layers "F.Cu" "B.Cu") (free yes) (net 3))
 (via (at 149.682 109.69) (size 0.6) (drill 0.3) (layers "F.Cu" "B.Cu") (free yes) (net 3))
 (via (at 152.73 109.69) (size 0.6) (drill 0.3) (layers "F.Cu" "B.Cu") (free yes) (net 3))
 (via (at 150.444 101.308) (size 0.6) (drill 0.3) (layers "F.Cu" "B.Cu") (free yes) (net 3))
 (via (at 150.444 109.69) (size 0.6) (drill 0.3) (layers "F.Cu" "B.Cu") (free yes) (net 3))
 (via (at 151.968 102.07) (size 0.6) (drill 0.3) (layers "F.Cu" "B.Cu") (free yes) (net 3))
 (via (at 147.396 108.928) (size 0.6) (drill 0.3) (layers "F.Cu" "B.Cu") (free yes) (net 3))
 (via (at 148.158 102.07) (size 0.6) (drill 0.3) (layers "F.Cu" "B.Cu") (free yes) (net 3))
 (via (at 148.158 110.452) (size 0.6) (drill 0.3) (layers "F.Cu" "B.Cu") (free yes) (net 3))
 (via (at 148.158 108.928) (size 0.6) (drill 0.3) (layers "F.Cu" "B.Cu") (free yes) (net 3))
 (via (at 148.158 100.546) (size 0.6) (drill 0.3) (layers "F.Cu" "B.Cu") (free yes) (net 3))
 (via (at 149.682 102.07) (size 0.6) (drill 0.3) (layers "F.Cu" "B.Cu") (free yes) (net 3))
 (via (at 151.968 110.452) (size 0.6) (drill 0.3) (layers "F.Cu" "B.Cu") (free yes) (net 3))
 (via (at 149.682 101.308) (size 0.6) (drill 0.3) (layers "F.Cu" "B.Cu") (free yes) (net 3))
 (via (at 147.396 100.546) (size 0.6) (drill 0.3) (layers "F.Cu" "B.Cu") (free yes) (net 3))
 (via (at 148.158 109.69) (size 0.6) (drill 0.3) (layers "F.Cu" "B.Cu") (free yes) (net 3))
 (via (at 152.73 100.546) (size 0.6) (drill 0.3) (layers "F.Cu" "B.Cu") (free yes) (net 3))
 (via (at 152.73 110.452) (size 0.6) (drill 0.3) (layers "F.Cu" "B.Cu") (free yes) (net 3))
 (via (at 148.92 101.308) (size 0.6) (drill 0.3) (layers "F.Cu" "B.Cu") (free yes) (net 3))
 (segment (start 70.18 79.45) (end 76.372 79.45) (width 2) (layer "F.Cu") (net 4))
 (segment (start 76.372 79.45) (end 76.506 79.316) (width 1.5) (layer "F.Cu") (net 4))
 (segment (start 70.18 79.45) (end 76.372 79.45) (width 2) (layer "B.Cu") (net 4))
 (segment (start 76.372 79.45) (end 76.506 79.316) (width 0.2) (layer "B.Cu") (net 4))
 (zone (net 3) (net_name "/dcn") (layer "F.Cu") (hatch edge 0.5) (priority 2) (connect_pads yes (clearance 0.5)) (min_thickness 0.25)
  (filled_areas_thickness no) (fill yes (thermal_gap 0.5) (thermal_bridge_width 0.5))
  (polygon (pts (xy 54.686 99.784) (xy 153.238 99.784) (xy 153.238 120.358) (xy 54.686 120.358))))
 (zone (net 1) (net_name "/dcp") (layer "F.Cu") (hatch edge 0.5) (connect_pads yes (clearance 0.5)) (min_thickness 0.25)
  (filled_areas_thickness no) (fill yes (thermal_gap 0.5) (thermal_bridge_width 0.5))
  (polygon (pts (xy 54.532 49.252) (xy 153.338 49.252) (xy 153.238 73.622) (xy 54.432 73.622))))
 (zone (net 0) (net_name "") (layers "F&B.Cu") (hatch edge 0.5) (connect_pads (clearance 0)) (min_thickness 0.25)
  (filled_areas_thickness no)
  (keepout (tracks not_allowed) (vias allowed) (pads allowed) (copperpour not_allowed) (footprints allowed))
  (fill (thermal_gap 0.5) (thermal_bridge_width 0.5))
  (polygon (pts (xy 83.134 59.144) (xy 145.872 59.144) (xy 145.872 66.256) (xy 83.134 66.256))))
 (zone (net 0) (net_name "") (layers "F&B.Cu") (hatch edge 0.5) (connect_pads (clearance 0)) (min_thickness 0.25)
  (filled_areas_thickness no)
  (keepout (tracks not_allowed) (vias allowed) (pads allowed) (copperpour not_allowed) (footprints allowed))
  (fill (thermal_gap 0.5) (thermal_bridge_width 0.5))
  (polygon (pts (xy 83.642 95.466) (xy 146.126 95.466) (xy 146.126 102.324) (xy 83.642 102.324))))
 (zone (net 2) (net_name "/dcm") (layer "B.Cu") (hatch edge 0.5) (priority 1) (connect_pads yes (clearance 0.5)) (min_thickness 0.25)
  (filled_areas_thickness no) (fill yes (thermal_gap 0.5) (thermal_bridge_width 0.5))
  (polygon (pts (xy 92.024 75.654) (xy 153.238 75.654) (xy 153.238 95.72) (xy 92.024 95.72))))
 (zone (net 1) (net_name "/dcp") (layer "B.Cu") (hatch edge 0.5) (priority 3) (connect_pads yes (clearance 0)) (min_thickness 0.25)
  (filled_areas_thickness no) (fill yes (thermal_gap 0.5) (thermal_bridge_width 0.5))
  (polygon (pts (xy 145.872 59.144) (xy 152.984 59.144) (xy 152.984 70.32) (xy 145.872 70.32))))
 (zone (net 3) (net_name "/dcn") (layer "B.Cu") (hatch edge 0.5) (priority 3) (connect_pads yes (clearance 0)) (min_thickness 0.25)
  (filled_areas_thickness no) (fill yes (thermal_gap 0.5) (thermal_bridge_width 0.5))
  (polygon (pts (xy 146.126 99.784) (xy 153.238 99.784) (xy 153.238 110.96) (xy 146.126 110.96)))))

